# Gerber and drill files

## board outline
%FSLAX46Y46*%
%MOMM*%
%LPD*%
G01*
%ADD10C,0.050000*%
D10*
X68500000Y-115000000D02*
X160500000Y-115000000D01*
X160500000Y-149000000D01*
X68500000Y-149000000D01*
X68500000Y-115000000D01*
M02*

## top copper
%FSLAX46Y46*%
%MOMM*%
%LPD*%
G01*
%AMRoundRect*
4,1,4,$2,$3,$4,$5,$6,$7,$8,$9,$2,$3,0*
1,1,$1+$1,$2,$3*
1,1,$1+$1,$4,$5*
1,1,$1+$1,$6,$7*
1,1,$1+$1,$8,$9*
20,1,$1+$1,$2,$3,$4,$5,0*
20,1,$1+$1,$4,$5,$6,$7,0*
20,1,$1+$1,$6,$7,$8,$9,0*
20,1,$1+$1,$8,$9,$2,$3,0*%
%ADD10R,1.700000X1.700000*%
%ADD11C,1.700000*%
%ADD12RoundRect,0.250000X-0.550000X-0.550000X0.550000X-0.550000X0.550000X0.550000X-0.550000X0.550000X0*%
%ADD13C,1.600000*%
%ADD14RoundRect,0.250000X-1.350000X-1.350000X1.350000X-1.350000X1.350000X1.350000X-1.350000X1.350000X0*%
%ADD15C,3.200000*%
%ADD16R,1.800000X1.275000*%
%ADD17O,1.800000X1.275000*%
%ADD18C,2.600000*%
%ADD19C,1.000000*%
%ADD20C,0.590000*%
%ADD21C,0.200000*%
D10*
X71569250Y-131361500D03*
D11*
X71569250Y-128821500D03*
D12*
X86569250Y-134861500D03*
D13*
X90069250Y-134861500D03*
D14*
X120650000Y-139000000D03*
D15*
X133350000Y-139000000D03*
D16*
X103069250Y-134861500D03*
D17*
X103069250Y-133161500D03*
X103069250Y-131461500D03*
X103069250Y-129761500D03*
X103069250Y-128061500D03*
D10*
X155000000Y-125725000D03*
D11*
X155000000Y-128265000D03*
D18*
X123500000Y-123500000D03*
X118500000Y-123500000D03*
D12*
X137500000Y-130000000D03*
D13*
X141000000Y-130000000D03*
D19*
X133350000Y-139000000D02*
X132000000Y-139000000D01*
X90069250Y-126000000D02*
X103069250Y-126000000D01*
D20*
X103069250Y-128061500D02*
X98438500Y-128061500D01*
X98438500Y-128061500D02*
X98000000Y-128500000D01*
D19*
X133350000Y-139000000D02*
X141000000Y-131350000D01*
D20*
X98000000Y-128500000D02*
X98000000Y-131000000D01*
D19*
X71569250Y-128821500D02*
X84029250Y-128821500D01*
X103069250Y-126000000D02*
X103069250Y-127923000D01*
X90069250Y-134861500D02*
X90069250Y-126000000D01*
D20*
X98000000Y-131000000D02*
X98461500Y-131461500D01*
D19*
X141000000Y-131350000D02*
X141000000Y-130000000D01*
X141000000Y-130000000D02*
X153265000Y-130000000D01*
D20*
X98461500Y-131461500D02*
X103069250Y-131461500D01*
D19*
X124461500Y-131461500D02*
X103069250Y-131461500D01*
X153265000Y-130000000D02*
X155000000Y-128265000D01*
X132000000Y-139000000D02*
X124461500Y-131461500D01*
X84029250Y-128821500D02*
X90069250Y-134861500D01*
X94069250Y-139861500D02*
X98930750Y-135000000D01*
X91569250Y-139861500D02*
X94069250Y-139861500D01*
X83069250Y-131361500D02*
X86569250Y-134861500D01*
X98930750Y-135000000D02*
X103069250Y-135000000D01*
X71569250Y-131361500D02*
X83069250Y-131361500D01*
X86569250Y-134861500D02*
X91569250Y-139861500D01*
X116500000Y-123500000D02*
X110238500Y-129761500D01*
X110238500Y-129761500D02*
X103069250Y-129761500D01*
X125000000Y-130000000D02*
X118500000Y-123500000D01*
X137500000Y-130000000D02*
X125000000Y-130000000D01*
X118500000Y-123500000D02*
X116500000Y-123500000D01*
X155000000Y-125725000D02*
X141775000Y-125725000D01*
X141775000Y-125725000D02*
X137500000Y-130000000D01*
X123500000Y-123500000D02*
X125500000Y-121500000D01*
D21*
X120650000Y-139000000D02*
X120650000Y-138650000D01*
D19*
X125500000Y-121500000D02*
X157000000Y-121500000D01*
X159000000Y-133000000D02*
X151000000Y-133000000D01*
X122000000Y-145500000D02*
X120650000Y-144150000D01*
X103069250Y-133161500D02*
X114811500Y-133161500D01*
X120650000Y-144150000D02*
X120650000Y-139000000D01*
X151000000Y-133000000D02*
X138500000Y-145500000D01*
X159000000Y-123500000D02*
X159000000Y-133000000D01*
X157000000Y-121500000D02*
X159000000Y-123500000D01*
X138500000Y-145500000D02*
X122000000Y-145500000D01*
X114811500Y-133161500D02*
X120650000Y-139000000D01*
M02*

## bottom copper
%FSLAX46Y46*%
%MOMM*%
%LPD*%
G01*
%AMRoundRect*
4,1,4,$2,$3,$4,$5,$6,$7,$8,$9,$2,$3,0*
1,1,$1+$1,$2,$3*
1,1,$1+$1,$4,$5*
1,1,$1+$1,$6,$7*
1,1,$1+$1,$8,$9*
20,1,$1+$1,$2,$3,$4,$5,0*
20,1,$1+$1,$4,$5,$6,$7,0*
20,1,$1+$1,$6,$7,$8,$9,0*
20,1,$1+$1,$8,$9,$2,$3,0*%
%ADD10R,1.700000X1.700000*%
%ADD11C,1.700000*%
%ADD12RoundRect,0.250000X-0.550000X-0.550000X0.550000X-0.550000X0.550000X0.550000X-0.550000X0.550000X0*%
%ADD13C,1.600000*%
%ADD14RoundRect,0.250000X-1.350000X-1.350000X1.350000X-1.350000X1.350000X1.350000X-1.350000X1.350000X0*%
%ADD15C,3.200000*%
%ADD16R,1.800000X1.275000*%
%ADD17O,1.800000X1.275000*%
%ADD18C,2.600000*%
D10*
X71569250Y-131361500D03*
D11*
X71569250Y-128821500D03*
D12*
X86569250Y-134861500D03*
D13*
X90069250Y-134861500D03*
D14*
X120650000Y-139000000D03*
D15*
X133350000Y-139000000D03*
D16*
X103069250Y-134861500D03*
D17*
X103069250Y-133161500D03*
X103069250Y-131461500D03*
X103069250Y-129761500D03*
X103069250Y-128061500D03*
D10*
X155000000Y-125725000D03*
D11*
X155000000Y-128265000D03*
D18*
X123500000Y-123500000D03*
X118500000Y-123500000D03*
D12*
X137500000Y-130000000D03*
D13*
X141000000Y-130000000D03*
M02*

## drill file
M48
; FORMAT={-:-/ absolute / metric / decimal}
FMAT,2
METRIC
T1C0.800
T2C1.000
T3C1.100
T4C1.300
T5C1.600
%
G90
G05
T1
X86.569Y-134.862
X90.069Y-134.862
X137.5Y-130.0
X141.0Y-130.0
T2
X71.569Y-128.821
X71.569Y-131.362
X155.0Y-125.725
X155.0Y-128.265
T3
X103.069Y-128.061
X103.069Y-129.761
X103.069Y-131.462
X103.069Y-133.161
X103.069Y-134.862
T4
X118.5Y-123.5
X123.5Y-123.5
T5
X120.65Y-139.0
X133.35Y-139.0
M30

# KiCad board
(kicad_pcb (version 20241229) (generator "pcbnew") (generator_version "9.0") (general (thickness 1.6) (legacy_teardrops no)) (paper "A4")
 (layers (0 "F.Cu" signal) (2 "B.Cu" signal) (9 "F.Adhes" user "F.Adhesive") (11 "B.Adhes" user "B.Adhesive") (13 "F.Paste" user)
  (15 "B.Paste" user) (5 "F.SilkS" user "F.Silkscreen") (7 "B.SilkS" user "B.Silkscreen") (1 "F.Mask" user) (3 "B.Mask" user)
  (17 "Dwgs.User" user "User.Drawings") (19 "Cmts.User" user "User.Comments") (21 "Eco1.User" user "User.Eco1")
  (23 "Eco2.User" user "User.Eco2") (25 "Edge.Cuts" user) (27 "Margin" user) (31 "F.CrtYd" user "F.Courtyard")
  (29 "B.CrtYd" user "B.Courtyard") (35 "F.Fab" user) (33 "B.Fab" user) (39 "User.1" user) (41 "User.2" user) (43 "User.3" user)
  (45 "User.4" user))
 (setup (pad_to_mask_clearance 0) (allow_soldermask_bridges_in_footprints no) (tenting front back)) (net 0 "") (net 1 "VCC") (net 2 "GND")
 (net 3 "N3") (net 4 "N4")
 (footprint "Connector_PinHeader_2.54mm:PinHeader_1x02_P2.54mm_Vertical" (layer "F.Cu") (at 71.56925 131.3615 180)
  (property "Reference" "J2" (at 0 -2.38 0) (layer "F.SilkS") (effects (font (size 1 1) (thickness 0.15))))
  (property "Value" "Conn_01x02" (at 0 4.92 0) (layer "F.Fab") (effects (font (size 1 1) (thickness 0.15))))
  (pad "1" thru_hole rect (at 0 0 180) (size 1.7 1.7) (drill 1) (layers "*.Cu" "*.Mask") (remove_unused_layers no) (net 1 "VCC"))
  (pad "2" thru_hole circle (at 0 2.54 180) (size 1.7 1.7) (drill 1) (layers "*.Cu" "*.Mask") (remove_unused_layers no) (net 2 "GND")))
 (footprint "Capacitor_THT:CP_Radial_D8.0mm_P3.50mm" (layer "F.Cu") (at 86.56925 134.8615)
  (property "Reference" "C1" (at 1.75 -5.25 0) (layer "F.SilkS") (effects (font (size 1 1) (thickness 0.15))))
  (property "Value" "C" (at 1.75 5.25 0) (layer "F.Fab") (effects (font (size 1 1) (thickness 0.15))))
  (pad "1" thru_hole roundrect (at 0 0) (size 1.6 1.6) (drill 0.8) (layers "*.Cu" "*.Mask") (remove_unused_layers no)
   (roundrect_rratio 0.15625) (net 1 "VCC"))
  (pad "2" thru_hole circle (at 3.5 0) (size 1.6 1.6) (drill 0.8) (layers "*.Cu" "*.Mask") (remove_unused_layers no) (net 2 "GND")))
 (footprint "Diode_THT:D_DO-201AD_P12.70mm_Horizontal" (layer "F.Cu") (at 120.65 139)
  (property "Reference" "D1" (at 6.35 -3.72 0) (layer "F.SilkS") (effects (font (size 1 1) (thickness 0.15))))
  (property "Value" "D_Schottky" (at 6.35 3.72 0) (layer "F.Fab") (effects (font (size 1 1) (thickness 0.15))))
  (pad "1" thru_hole roundrect (at 0 0) (size 3.2 3.2) (drill 1.6) (layers "*.Cu" "*.Mask") (remove_unused_layers no)
   (roundrect_rratio 0.078125) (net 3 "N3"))
  (pad "2" thru_hole circle (at 12.7 0) (size 3.2 3.2) (drill 1.6) (layers "*.Cu" "*.Mask") (remove_unused_layers no) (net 2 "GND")))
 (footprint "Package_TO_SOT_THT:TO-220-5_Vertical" (layer "F.Cu") (at 103.06925 134.8615 90)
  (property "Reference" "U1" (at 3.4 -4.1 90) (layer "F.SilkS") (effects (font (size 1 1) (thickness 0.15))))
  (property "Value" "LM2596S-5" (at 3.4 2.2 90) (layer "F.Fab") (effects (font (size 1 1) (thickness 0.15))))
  (pad "1" thru_hole rect (at 0 0 90) (size 1.275 1.8) (drill 1.1) (layers "*.Cu" "*.Mask") (remove_unused_layers no) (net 1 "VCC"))
  (pad "2" thru_hole oval (at 1.7 0 90) (size 1.275 1.8) (drill 1.1) (layers "*.Cu" "*.Mask") (remove_unused_layers no) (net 3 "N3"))
  (pad "3" thru_hole oval (at 3.4 0 90) (size 1.275 1.8) (drill 1.1) (layers "*.Cu" "*.Mask") (remove_unused_layers no) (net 2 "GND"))
  (pad "4" thru_hole oval (at 5.1 0 90) (size 1.275 1.8) (drill 1.1) (layers "*.Cu" "*.Mask") (remove_unused_layers no) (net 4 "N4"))
  (pad "5" thru_hole oval (at 6.8 0 90) (size 1.275 1.8) (drill 1.1) (layers "*.Cu" "*.Mask") (remove_unused_layers no) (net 2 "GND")))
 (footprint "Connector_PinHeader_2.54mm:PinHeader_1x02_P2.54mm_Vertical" (layer "F.Cu") (at 155 125.725)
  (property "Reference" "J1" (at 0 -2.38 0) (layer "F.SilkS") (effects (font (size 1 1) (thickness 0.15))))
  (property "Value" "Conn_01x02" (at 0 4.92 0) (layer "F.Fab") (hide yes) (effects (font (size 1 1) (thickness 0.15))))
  (pad "1" thru_hole rect (at 0 0) (size 1.7 1.7) (drill 1) (layers "*.Cu" "*.Mask") (remove_unused_layers no) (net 4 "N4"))
  (pad "2" thru_hole circle (at 0 2.54) (size 1.7 1.7) (drill 1) (layers "*.Cu" "*.Mask") (remove_unused_layers no) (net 2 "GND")))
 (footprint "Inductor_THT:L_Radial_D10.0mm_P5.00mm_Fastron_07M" (layer "F.Cu") (at 123.5 123.5 180)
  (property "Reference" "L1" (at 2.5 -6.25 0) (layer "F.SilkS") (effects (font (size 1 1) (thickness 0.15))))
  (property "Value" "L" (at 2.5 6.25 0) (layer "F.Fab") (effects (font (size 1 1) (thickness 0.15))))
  (pad "1" thru_hole circle (at 0 0 180) (size 2.6 2.6) (drill 1.3) (layers "*.Cu" "*.Mask") (remove_unused_layers no) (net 3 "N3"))
  (pad "2" thru_hole circle (at 5 0 180) (size 2.6 2.6) (drill 1.3) (layers "*.Cu" "*.Mask") (remove_unused_layers no) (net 4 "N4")))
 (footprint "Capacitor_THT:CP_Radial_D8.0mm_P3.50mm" (layer "F.Cu") (at 137.5 130)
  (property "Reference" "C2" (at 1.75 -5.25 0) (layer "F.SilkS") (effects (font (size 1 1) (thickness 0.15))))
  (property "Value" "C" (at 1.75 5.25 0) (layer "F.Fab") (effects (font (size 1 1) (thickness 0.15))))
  (pad "1" thru_hole roundrect (at 0 0) (size 1.6 1.6) (drill 0.8) (layers "*.Cu" "*.Mask") (remove_unused_layers no)
   (roundrect_rratio 0.15625) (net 4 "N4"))
  (pad "2" thru_hole circle (at 3.5 0) (size 1.6 1.6) (drill 0.8) (layers "*.Cu" "*.Mask") (remove_unused_layers no) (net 2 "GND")))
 (gr_rect (start 68.5 115) (end 160.5 149) (stroke (width 0.05) (type default)) (fill no) (layer "Edge.Cuts"))
 (segment (start 133.35 139) (end 132 139) (width 1) (layer "F.Cu") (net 2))
 (segment (start 90.06925 126) (end 103.06925 126) (width 1) (layer "F.Cu") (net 2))
 (segment (start 103.06925 128.0615) (end 98.4385 128.0615) (width 0.59) (layer "F.Cu") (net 2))
 (segment (start 98.4385 128.0615) (end 98 128.5) (width 0.59) (layer "F.Cu") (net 2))
 (segment (start 133.35 139) (end 141 131.35) (width 1) (layer "F.Cu") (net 2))
 (segment (start 98 128.5) (end 98 131) (width 0.59) (layer "F.Cu") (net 2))
 (segment (start 71.56925 128.8215) (end 84.02925 128.8215) (width 1) (layer "F.Cu") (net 2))
 (segment (start 103.06925 126) (end 103.06925 127.923) (width 1) (layer "F.Cu") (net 2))
 (segment (start 90.06925 134.8615) (end 90.06925 126) (width 1) (layer "F.Cu") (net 2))
 (segment (start 98 131) (end 98.4615 131.4615) (width 0.59) (layer "F.Cu") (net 2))
 (segment (start 141 131.35) (end 141 130) (width 1) (layer "F.Cu") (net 2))
 (segment (start 141 130) (end 153.265 130) (width 1) (layer "F.Cu") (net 2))
 (segment (start 98.4615 131.4615) (end 103.06925 131.4615) (width 0.59) (layer "F.Cu") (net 2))
 (segment (start 124.4615 131.4615) (end 103.06925 131.4615) (width 1) (layer "F.Cu") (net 2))
 (segment (start 153.265 130) (end 155 128.265) (width 1) (layer "F.Cu") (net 2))
 (segment (start 132 139) (end 124.4615 131.4615) (width 1) (layer "F.Cu") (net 2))
 (segment (start 84.02925 128.8215) (end 90.06925 134.8615) (width 1) (layer "F.Cu") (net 2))
 (segment (start 94.06925 139.8615) (end 98.93075 135) (width 1) (layer "F.Cu") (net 1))
 (segment (start 91.56925 139.8615) (end 94.06925 139.8615) (width 1) (layer "F.Cu") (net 1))
 (segment (start 83.06925 131.3615) (end 86.56925 134.8615) (width 1) (layer "F.Cu") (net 1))
 (segment (start 98.93075 135) (end 103.06925 135) (width 1) (layer "F.Cu") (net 1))
 (segment (start 71.56925 131.3615) (end 83.06925 131.3615) (width 1) (layer "F.Cu") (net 1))
 (segment (start 86.56925 134.8615) (end 91.56925 139.8615) (width 1) (layer "F.Cu") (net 1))
 (segment (start 116.5 123.5) (end 110.2385 129.7615) (width 1) (layer "F.Cu") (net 4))
 (segment (start 110.2385 129.7615) (end 103.06925 129.7615) (width 1) (layer "F.Cu") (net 4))
 (segment (start 125 130) (end 118.5 123.5) (width 1) (layer "F.Cu") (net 4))
 (segment (start 137.5 130) (end 125 130) (width 1) (layer "F.Cu") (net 4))
 (segment (start 118.5 123.5) (end 116.5 123.5) (width 1) (layer "F.Cu") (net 4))
 (segment (start 155 125.725) (end 141.775 125.725) (width 1) (layer "F.Cu") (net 4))
 (segment (start 141.775 125.725) (end 137.5 130) (width 1) (layer "F.Cu") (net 4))
 (segment (start 123.5 123.5) (end 125.5 121.5) (width 1) (layer "F.Cu") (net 3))
 (segment (start 120.65 139) (end 120.65 138.65) (width 0.2) (layer "F.Cu") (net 3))
 (segment (start 125.5 121.5) (end 157 121.5) (width 1) (layer "F.Cu") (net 3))
 (segment (start 159 133) (end 151 133) (width 1) (layer "F.Cu") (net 3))
 (segment (start 122 145.5) (end 120.65 144.15) (width 1) (layer "F.Cu") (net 3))
 (segment (start 103.06925 133.1615) (end 114.8115 133.1615) (width 1) (layer "F.Cu") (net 3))
 (segment (start 120.65 144.15) (end 120.65 139) (width 1) (layer "F.Cu") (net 3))
 (segment (start 151 133) (end 138.5 145.5) (width 1) (layer "F.Cu") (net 3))
 (segment (start 159 123.5) (end 159 133) (width 1) (layer "F.Cu") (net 3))
 (segment (start 157 121.5) (end 159 123.5) (width 1) (layer "F.Cu") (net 3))
 (segment (start 138.5 145.5) (end 122 145.5) (width 1) (layer "F.Cu") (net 3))
 (segment (start 114.8115 133.1615) (end 120.65 139) (width 1) (layer "F.Cu") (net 3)))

